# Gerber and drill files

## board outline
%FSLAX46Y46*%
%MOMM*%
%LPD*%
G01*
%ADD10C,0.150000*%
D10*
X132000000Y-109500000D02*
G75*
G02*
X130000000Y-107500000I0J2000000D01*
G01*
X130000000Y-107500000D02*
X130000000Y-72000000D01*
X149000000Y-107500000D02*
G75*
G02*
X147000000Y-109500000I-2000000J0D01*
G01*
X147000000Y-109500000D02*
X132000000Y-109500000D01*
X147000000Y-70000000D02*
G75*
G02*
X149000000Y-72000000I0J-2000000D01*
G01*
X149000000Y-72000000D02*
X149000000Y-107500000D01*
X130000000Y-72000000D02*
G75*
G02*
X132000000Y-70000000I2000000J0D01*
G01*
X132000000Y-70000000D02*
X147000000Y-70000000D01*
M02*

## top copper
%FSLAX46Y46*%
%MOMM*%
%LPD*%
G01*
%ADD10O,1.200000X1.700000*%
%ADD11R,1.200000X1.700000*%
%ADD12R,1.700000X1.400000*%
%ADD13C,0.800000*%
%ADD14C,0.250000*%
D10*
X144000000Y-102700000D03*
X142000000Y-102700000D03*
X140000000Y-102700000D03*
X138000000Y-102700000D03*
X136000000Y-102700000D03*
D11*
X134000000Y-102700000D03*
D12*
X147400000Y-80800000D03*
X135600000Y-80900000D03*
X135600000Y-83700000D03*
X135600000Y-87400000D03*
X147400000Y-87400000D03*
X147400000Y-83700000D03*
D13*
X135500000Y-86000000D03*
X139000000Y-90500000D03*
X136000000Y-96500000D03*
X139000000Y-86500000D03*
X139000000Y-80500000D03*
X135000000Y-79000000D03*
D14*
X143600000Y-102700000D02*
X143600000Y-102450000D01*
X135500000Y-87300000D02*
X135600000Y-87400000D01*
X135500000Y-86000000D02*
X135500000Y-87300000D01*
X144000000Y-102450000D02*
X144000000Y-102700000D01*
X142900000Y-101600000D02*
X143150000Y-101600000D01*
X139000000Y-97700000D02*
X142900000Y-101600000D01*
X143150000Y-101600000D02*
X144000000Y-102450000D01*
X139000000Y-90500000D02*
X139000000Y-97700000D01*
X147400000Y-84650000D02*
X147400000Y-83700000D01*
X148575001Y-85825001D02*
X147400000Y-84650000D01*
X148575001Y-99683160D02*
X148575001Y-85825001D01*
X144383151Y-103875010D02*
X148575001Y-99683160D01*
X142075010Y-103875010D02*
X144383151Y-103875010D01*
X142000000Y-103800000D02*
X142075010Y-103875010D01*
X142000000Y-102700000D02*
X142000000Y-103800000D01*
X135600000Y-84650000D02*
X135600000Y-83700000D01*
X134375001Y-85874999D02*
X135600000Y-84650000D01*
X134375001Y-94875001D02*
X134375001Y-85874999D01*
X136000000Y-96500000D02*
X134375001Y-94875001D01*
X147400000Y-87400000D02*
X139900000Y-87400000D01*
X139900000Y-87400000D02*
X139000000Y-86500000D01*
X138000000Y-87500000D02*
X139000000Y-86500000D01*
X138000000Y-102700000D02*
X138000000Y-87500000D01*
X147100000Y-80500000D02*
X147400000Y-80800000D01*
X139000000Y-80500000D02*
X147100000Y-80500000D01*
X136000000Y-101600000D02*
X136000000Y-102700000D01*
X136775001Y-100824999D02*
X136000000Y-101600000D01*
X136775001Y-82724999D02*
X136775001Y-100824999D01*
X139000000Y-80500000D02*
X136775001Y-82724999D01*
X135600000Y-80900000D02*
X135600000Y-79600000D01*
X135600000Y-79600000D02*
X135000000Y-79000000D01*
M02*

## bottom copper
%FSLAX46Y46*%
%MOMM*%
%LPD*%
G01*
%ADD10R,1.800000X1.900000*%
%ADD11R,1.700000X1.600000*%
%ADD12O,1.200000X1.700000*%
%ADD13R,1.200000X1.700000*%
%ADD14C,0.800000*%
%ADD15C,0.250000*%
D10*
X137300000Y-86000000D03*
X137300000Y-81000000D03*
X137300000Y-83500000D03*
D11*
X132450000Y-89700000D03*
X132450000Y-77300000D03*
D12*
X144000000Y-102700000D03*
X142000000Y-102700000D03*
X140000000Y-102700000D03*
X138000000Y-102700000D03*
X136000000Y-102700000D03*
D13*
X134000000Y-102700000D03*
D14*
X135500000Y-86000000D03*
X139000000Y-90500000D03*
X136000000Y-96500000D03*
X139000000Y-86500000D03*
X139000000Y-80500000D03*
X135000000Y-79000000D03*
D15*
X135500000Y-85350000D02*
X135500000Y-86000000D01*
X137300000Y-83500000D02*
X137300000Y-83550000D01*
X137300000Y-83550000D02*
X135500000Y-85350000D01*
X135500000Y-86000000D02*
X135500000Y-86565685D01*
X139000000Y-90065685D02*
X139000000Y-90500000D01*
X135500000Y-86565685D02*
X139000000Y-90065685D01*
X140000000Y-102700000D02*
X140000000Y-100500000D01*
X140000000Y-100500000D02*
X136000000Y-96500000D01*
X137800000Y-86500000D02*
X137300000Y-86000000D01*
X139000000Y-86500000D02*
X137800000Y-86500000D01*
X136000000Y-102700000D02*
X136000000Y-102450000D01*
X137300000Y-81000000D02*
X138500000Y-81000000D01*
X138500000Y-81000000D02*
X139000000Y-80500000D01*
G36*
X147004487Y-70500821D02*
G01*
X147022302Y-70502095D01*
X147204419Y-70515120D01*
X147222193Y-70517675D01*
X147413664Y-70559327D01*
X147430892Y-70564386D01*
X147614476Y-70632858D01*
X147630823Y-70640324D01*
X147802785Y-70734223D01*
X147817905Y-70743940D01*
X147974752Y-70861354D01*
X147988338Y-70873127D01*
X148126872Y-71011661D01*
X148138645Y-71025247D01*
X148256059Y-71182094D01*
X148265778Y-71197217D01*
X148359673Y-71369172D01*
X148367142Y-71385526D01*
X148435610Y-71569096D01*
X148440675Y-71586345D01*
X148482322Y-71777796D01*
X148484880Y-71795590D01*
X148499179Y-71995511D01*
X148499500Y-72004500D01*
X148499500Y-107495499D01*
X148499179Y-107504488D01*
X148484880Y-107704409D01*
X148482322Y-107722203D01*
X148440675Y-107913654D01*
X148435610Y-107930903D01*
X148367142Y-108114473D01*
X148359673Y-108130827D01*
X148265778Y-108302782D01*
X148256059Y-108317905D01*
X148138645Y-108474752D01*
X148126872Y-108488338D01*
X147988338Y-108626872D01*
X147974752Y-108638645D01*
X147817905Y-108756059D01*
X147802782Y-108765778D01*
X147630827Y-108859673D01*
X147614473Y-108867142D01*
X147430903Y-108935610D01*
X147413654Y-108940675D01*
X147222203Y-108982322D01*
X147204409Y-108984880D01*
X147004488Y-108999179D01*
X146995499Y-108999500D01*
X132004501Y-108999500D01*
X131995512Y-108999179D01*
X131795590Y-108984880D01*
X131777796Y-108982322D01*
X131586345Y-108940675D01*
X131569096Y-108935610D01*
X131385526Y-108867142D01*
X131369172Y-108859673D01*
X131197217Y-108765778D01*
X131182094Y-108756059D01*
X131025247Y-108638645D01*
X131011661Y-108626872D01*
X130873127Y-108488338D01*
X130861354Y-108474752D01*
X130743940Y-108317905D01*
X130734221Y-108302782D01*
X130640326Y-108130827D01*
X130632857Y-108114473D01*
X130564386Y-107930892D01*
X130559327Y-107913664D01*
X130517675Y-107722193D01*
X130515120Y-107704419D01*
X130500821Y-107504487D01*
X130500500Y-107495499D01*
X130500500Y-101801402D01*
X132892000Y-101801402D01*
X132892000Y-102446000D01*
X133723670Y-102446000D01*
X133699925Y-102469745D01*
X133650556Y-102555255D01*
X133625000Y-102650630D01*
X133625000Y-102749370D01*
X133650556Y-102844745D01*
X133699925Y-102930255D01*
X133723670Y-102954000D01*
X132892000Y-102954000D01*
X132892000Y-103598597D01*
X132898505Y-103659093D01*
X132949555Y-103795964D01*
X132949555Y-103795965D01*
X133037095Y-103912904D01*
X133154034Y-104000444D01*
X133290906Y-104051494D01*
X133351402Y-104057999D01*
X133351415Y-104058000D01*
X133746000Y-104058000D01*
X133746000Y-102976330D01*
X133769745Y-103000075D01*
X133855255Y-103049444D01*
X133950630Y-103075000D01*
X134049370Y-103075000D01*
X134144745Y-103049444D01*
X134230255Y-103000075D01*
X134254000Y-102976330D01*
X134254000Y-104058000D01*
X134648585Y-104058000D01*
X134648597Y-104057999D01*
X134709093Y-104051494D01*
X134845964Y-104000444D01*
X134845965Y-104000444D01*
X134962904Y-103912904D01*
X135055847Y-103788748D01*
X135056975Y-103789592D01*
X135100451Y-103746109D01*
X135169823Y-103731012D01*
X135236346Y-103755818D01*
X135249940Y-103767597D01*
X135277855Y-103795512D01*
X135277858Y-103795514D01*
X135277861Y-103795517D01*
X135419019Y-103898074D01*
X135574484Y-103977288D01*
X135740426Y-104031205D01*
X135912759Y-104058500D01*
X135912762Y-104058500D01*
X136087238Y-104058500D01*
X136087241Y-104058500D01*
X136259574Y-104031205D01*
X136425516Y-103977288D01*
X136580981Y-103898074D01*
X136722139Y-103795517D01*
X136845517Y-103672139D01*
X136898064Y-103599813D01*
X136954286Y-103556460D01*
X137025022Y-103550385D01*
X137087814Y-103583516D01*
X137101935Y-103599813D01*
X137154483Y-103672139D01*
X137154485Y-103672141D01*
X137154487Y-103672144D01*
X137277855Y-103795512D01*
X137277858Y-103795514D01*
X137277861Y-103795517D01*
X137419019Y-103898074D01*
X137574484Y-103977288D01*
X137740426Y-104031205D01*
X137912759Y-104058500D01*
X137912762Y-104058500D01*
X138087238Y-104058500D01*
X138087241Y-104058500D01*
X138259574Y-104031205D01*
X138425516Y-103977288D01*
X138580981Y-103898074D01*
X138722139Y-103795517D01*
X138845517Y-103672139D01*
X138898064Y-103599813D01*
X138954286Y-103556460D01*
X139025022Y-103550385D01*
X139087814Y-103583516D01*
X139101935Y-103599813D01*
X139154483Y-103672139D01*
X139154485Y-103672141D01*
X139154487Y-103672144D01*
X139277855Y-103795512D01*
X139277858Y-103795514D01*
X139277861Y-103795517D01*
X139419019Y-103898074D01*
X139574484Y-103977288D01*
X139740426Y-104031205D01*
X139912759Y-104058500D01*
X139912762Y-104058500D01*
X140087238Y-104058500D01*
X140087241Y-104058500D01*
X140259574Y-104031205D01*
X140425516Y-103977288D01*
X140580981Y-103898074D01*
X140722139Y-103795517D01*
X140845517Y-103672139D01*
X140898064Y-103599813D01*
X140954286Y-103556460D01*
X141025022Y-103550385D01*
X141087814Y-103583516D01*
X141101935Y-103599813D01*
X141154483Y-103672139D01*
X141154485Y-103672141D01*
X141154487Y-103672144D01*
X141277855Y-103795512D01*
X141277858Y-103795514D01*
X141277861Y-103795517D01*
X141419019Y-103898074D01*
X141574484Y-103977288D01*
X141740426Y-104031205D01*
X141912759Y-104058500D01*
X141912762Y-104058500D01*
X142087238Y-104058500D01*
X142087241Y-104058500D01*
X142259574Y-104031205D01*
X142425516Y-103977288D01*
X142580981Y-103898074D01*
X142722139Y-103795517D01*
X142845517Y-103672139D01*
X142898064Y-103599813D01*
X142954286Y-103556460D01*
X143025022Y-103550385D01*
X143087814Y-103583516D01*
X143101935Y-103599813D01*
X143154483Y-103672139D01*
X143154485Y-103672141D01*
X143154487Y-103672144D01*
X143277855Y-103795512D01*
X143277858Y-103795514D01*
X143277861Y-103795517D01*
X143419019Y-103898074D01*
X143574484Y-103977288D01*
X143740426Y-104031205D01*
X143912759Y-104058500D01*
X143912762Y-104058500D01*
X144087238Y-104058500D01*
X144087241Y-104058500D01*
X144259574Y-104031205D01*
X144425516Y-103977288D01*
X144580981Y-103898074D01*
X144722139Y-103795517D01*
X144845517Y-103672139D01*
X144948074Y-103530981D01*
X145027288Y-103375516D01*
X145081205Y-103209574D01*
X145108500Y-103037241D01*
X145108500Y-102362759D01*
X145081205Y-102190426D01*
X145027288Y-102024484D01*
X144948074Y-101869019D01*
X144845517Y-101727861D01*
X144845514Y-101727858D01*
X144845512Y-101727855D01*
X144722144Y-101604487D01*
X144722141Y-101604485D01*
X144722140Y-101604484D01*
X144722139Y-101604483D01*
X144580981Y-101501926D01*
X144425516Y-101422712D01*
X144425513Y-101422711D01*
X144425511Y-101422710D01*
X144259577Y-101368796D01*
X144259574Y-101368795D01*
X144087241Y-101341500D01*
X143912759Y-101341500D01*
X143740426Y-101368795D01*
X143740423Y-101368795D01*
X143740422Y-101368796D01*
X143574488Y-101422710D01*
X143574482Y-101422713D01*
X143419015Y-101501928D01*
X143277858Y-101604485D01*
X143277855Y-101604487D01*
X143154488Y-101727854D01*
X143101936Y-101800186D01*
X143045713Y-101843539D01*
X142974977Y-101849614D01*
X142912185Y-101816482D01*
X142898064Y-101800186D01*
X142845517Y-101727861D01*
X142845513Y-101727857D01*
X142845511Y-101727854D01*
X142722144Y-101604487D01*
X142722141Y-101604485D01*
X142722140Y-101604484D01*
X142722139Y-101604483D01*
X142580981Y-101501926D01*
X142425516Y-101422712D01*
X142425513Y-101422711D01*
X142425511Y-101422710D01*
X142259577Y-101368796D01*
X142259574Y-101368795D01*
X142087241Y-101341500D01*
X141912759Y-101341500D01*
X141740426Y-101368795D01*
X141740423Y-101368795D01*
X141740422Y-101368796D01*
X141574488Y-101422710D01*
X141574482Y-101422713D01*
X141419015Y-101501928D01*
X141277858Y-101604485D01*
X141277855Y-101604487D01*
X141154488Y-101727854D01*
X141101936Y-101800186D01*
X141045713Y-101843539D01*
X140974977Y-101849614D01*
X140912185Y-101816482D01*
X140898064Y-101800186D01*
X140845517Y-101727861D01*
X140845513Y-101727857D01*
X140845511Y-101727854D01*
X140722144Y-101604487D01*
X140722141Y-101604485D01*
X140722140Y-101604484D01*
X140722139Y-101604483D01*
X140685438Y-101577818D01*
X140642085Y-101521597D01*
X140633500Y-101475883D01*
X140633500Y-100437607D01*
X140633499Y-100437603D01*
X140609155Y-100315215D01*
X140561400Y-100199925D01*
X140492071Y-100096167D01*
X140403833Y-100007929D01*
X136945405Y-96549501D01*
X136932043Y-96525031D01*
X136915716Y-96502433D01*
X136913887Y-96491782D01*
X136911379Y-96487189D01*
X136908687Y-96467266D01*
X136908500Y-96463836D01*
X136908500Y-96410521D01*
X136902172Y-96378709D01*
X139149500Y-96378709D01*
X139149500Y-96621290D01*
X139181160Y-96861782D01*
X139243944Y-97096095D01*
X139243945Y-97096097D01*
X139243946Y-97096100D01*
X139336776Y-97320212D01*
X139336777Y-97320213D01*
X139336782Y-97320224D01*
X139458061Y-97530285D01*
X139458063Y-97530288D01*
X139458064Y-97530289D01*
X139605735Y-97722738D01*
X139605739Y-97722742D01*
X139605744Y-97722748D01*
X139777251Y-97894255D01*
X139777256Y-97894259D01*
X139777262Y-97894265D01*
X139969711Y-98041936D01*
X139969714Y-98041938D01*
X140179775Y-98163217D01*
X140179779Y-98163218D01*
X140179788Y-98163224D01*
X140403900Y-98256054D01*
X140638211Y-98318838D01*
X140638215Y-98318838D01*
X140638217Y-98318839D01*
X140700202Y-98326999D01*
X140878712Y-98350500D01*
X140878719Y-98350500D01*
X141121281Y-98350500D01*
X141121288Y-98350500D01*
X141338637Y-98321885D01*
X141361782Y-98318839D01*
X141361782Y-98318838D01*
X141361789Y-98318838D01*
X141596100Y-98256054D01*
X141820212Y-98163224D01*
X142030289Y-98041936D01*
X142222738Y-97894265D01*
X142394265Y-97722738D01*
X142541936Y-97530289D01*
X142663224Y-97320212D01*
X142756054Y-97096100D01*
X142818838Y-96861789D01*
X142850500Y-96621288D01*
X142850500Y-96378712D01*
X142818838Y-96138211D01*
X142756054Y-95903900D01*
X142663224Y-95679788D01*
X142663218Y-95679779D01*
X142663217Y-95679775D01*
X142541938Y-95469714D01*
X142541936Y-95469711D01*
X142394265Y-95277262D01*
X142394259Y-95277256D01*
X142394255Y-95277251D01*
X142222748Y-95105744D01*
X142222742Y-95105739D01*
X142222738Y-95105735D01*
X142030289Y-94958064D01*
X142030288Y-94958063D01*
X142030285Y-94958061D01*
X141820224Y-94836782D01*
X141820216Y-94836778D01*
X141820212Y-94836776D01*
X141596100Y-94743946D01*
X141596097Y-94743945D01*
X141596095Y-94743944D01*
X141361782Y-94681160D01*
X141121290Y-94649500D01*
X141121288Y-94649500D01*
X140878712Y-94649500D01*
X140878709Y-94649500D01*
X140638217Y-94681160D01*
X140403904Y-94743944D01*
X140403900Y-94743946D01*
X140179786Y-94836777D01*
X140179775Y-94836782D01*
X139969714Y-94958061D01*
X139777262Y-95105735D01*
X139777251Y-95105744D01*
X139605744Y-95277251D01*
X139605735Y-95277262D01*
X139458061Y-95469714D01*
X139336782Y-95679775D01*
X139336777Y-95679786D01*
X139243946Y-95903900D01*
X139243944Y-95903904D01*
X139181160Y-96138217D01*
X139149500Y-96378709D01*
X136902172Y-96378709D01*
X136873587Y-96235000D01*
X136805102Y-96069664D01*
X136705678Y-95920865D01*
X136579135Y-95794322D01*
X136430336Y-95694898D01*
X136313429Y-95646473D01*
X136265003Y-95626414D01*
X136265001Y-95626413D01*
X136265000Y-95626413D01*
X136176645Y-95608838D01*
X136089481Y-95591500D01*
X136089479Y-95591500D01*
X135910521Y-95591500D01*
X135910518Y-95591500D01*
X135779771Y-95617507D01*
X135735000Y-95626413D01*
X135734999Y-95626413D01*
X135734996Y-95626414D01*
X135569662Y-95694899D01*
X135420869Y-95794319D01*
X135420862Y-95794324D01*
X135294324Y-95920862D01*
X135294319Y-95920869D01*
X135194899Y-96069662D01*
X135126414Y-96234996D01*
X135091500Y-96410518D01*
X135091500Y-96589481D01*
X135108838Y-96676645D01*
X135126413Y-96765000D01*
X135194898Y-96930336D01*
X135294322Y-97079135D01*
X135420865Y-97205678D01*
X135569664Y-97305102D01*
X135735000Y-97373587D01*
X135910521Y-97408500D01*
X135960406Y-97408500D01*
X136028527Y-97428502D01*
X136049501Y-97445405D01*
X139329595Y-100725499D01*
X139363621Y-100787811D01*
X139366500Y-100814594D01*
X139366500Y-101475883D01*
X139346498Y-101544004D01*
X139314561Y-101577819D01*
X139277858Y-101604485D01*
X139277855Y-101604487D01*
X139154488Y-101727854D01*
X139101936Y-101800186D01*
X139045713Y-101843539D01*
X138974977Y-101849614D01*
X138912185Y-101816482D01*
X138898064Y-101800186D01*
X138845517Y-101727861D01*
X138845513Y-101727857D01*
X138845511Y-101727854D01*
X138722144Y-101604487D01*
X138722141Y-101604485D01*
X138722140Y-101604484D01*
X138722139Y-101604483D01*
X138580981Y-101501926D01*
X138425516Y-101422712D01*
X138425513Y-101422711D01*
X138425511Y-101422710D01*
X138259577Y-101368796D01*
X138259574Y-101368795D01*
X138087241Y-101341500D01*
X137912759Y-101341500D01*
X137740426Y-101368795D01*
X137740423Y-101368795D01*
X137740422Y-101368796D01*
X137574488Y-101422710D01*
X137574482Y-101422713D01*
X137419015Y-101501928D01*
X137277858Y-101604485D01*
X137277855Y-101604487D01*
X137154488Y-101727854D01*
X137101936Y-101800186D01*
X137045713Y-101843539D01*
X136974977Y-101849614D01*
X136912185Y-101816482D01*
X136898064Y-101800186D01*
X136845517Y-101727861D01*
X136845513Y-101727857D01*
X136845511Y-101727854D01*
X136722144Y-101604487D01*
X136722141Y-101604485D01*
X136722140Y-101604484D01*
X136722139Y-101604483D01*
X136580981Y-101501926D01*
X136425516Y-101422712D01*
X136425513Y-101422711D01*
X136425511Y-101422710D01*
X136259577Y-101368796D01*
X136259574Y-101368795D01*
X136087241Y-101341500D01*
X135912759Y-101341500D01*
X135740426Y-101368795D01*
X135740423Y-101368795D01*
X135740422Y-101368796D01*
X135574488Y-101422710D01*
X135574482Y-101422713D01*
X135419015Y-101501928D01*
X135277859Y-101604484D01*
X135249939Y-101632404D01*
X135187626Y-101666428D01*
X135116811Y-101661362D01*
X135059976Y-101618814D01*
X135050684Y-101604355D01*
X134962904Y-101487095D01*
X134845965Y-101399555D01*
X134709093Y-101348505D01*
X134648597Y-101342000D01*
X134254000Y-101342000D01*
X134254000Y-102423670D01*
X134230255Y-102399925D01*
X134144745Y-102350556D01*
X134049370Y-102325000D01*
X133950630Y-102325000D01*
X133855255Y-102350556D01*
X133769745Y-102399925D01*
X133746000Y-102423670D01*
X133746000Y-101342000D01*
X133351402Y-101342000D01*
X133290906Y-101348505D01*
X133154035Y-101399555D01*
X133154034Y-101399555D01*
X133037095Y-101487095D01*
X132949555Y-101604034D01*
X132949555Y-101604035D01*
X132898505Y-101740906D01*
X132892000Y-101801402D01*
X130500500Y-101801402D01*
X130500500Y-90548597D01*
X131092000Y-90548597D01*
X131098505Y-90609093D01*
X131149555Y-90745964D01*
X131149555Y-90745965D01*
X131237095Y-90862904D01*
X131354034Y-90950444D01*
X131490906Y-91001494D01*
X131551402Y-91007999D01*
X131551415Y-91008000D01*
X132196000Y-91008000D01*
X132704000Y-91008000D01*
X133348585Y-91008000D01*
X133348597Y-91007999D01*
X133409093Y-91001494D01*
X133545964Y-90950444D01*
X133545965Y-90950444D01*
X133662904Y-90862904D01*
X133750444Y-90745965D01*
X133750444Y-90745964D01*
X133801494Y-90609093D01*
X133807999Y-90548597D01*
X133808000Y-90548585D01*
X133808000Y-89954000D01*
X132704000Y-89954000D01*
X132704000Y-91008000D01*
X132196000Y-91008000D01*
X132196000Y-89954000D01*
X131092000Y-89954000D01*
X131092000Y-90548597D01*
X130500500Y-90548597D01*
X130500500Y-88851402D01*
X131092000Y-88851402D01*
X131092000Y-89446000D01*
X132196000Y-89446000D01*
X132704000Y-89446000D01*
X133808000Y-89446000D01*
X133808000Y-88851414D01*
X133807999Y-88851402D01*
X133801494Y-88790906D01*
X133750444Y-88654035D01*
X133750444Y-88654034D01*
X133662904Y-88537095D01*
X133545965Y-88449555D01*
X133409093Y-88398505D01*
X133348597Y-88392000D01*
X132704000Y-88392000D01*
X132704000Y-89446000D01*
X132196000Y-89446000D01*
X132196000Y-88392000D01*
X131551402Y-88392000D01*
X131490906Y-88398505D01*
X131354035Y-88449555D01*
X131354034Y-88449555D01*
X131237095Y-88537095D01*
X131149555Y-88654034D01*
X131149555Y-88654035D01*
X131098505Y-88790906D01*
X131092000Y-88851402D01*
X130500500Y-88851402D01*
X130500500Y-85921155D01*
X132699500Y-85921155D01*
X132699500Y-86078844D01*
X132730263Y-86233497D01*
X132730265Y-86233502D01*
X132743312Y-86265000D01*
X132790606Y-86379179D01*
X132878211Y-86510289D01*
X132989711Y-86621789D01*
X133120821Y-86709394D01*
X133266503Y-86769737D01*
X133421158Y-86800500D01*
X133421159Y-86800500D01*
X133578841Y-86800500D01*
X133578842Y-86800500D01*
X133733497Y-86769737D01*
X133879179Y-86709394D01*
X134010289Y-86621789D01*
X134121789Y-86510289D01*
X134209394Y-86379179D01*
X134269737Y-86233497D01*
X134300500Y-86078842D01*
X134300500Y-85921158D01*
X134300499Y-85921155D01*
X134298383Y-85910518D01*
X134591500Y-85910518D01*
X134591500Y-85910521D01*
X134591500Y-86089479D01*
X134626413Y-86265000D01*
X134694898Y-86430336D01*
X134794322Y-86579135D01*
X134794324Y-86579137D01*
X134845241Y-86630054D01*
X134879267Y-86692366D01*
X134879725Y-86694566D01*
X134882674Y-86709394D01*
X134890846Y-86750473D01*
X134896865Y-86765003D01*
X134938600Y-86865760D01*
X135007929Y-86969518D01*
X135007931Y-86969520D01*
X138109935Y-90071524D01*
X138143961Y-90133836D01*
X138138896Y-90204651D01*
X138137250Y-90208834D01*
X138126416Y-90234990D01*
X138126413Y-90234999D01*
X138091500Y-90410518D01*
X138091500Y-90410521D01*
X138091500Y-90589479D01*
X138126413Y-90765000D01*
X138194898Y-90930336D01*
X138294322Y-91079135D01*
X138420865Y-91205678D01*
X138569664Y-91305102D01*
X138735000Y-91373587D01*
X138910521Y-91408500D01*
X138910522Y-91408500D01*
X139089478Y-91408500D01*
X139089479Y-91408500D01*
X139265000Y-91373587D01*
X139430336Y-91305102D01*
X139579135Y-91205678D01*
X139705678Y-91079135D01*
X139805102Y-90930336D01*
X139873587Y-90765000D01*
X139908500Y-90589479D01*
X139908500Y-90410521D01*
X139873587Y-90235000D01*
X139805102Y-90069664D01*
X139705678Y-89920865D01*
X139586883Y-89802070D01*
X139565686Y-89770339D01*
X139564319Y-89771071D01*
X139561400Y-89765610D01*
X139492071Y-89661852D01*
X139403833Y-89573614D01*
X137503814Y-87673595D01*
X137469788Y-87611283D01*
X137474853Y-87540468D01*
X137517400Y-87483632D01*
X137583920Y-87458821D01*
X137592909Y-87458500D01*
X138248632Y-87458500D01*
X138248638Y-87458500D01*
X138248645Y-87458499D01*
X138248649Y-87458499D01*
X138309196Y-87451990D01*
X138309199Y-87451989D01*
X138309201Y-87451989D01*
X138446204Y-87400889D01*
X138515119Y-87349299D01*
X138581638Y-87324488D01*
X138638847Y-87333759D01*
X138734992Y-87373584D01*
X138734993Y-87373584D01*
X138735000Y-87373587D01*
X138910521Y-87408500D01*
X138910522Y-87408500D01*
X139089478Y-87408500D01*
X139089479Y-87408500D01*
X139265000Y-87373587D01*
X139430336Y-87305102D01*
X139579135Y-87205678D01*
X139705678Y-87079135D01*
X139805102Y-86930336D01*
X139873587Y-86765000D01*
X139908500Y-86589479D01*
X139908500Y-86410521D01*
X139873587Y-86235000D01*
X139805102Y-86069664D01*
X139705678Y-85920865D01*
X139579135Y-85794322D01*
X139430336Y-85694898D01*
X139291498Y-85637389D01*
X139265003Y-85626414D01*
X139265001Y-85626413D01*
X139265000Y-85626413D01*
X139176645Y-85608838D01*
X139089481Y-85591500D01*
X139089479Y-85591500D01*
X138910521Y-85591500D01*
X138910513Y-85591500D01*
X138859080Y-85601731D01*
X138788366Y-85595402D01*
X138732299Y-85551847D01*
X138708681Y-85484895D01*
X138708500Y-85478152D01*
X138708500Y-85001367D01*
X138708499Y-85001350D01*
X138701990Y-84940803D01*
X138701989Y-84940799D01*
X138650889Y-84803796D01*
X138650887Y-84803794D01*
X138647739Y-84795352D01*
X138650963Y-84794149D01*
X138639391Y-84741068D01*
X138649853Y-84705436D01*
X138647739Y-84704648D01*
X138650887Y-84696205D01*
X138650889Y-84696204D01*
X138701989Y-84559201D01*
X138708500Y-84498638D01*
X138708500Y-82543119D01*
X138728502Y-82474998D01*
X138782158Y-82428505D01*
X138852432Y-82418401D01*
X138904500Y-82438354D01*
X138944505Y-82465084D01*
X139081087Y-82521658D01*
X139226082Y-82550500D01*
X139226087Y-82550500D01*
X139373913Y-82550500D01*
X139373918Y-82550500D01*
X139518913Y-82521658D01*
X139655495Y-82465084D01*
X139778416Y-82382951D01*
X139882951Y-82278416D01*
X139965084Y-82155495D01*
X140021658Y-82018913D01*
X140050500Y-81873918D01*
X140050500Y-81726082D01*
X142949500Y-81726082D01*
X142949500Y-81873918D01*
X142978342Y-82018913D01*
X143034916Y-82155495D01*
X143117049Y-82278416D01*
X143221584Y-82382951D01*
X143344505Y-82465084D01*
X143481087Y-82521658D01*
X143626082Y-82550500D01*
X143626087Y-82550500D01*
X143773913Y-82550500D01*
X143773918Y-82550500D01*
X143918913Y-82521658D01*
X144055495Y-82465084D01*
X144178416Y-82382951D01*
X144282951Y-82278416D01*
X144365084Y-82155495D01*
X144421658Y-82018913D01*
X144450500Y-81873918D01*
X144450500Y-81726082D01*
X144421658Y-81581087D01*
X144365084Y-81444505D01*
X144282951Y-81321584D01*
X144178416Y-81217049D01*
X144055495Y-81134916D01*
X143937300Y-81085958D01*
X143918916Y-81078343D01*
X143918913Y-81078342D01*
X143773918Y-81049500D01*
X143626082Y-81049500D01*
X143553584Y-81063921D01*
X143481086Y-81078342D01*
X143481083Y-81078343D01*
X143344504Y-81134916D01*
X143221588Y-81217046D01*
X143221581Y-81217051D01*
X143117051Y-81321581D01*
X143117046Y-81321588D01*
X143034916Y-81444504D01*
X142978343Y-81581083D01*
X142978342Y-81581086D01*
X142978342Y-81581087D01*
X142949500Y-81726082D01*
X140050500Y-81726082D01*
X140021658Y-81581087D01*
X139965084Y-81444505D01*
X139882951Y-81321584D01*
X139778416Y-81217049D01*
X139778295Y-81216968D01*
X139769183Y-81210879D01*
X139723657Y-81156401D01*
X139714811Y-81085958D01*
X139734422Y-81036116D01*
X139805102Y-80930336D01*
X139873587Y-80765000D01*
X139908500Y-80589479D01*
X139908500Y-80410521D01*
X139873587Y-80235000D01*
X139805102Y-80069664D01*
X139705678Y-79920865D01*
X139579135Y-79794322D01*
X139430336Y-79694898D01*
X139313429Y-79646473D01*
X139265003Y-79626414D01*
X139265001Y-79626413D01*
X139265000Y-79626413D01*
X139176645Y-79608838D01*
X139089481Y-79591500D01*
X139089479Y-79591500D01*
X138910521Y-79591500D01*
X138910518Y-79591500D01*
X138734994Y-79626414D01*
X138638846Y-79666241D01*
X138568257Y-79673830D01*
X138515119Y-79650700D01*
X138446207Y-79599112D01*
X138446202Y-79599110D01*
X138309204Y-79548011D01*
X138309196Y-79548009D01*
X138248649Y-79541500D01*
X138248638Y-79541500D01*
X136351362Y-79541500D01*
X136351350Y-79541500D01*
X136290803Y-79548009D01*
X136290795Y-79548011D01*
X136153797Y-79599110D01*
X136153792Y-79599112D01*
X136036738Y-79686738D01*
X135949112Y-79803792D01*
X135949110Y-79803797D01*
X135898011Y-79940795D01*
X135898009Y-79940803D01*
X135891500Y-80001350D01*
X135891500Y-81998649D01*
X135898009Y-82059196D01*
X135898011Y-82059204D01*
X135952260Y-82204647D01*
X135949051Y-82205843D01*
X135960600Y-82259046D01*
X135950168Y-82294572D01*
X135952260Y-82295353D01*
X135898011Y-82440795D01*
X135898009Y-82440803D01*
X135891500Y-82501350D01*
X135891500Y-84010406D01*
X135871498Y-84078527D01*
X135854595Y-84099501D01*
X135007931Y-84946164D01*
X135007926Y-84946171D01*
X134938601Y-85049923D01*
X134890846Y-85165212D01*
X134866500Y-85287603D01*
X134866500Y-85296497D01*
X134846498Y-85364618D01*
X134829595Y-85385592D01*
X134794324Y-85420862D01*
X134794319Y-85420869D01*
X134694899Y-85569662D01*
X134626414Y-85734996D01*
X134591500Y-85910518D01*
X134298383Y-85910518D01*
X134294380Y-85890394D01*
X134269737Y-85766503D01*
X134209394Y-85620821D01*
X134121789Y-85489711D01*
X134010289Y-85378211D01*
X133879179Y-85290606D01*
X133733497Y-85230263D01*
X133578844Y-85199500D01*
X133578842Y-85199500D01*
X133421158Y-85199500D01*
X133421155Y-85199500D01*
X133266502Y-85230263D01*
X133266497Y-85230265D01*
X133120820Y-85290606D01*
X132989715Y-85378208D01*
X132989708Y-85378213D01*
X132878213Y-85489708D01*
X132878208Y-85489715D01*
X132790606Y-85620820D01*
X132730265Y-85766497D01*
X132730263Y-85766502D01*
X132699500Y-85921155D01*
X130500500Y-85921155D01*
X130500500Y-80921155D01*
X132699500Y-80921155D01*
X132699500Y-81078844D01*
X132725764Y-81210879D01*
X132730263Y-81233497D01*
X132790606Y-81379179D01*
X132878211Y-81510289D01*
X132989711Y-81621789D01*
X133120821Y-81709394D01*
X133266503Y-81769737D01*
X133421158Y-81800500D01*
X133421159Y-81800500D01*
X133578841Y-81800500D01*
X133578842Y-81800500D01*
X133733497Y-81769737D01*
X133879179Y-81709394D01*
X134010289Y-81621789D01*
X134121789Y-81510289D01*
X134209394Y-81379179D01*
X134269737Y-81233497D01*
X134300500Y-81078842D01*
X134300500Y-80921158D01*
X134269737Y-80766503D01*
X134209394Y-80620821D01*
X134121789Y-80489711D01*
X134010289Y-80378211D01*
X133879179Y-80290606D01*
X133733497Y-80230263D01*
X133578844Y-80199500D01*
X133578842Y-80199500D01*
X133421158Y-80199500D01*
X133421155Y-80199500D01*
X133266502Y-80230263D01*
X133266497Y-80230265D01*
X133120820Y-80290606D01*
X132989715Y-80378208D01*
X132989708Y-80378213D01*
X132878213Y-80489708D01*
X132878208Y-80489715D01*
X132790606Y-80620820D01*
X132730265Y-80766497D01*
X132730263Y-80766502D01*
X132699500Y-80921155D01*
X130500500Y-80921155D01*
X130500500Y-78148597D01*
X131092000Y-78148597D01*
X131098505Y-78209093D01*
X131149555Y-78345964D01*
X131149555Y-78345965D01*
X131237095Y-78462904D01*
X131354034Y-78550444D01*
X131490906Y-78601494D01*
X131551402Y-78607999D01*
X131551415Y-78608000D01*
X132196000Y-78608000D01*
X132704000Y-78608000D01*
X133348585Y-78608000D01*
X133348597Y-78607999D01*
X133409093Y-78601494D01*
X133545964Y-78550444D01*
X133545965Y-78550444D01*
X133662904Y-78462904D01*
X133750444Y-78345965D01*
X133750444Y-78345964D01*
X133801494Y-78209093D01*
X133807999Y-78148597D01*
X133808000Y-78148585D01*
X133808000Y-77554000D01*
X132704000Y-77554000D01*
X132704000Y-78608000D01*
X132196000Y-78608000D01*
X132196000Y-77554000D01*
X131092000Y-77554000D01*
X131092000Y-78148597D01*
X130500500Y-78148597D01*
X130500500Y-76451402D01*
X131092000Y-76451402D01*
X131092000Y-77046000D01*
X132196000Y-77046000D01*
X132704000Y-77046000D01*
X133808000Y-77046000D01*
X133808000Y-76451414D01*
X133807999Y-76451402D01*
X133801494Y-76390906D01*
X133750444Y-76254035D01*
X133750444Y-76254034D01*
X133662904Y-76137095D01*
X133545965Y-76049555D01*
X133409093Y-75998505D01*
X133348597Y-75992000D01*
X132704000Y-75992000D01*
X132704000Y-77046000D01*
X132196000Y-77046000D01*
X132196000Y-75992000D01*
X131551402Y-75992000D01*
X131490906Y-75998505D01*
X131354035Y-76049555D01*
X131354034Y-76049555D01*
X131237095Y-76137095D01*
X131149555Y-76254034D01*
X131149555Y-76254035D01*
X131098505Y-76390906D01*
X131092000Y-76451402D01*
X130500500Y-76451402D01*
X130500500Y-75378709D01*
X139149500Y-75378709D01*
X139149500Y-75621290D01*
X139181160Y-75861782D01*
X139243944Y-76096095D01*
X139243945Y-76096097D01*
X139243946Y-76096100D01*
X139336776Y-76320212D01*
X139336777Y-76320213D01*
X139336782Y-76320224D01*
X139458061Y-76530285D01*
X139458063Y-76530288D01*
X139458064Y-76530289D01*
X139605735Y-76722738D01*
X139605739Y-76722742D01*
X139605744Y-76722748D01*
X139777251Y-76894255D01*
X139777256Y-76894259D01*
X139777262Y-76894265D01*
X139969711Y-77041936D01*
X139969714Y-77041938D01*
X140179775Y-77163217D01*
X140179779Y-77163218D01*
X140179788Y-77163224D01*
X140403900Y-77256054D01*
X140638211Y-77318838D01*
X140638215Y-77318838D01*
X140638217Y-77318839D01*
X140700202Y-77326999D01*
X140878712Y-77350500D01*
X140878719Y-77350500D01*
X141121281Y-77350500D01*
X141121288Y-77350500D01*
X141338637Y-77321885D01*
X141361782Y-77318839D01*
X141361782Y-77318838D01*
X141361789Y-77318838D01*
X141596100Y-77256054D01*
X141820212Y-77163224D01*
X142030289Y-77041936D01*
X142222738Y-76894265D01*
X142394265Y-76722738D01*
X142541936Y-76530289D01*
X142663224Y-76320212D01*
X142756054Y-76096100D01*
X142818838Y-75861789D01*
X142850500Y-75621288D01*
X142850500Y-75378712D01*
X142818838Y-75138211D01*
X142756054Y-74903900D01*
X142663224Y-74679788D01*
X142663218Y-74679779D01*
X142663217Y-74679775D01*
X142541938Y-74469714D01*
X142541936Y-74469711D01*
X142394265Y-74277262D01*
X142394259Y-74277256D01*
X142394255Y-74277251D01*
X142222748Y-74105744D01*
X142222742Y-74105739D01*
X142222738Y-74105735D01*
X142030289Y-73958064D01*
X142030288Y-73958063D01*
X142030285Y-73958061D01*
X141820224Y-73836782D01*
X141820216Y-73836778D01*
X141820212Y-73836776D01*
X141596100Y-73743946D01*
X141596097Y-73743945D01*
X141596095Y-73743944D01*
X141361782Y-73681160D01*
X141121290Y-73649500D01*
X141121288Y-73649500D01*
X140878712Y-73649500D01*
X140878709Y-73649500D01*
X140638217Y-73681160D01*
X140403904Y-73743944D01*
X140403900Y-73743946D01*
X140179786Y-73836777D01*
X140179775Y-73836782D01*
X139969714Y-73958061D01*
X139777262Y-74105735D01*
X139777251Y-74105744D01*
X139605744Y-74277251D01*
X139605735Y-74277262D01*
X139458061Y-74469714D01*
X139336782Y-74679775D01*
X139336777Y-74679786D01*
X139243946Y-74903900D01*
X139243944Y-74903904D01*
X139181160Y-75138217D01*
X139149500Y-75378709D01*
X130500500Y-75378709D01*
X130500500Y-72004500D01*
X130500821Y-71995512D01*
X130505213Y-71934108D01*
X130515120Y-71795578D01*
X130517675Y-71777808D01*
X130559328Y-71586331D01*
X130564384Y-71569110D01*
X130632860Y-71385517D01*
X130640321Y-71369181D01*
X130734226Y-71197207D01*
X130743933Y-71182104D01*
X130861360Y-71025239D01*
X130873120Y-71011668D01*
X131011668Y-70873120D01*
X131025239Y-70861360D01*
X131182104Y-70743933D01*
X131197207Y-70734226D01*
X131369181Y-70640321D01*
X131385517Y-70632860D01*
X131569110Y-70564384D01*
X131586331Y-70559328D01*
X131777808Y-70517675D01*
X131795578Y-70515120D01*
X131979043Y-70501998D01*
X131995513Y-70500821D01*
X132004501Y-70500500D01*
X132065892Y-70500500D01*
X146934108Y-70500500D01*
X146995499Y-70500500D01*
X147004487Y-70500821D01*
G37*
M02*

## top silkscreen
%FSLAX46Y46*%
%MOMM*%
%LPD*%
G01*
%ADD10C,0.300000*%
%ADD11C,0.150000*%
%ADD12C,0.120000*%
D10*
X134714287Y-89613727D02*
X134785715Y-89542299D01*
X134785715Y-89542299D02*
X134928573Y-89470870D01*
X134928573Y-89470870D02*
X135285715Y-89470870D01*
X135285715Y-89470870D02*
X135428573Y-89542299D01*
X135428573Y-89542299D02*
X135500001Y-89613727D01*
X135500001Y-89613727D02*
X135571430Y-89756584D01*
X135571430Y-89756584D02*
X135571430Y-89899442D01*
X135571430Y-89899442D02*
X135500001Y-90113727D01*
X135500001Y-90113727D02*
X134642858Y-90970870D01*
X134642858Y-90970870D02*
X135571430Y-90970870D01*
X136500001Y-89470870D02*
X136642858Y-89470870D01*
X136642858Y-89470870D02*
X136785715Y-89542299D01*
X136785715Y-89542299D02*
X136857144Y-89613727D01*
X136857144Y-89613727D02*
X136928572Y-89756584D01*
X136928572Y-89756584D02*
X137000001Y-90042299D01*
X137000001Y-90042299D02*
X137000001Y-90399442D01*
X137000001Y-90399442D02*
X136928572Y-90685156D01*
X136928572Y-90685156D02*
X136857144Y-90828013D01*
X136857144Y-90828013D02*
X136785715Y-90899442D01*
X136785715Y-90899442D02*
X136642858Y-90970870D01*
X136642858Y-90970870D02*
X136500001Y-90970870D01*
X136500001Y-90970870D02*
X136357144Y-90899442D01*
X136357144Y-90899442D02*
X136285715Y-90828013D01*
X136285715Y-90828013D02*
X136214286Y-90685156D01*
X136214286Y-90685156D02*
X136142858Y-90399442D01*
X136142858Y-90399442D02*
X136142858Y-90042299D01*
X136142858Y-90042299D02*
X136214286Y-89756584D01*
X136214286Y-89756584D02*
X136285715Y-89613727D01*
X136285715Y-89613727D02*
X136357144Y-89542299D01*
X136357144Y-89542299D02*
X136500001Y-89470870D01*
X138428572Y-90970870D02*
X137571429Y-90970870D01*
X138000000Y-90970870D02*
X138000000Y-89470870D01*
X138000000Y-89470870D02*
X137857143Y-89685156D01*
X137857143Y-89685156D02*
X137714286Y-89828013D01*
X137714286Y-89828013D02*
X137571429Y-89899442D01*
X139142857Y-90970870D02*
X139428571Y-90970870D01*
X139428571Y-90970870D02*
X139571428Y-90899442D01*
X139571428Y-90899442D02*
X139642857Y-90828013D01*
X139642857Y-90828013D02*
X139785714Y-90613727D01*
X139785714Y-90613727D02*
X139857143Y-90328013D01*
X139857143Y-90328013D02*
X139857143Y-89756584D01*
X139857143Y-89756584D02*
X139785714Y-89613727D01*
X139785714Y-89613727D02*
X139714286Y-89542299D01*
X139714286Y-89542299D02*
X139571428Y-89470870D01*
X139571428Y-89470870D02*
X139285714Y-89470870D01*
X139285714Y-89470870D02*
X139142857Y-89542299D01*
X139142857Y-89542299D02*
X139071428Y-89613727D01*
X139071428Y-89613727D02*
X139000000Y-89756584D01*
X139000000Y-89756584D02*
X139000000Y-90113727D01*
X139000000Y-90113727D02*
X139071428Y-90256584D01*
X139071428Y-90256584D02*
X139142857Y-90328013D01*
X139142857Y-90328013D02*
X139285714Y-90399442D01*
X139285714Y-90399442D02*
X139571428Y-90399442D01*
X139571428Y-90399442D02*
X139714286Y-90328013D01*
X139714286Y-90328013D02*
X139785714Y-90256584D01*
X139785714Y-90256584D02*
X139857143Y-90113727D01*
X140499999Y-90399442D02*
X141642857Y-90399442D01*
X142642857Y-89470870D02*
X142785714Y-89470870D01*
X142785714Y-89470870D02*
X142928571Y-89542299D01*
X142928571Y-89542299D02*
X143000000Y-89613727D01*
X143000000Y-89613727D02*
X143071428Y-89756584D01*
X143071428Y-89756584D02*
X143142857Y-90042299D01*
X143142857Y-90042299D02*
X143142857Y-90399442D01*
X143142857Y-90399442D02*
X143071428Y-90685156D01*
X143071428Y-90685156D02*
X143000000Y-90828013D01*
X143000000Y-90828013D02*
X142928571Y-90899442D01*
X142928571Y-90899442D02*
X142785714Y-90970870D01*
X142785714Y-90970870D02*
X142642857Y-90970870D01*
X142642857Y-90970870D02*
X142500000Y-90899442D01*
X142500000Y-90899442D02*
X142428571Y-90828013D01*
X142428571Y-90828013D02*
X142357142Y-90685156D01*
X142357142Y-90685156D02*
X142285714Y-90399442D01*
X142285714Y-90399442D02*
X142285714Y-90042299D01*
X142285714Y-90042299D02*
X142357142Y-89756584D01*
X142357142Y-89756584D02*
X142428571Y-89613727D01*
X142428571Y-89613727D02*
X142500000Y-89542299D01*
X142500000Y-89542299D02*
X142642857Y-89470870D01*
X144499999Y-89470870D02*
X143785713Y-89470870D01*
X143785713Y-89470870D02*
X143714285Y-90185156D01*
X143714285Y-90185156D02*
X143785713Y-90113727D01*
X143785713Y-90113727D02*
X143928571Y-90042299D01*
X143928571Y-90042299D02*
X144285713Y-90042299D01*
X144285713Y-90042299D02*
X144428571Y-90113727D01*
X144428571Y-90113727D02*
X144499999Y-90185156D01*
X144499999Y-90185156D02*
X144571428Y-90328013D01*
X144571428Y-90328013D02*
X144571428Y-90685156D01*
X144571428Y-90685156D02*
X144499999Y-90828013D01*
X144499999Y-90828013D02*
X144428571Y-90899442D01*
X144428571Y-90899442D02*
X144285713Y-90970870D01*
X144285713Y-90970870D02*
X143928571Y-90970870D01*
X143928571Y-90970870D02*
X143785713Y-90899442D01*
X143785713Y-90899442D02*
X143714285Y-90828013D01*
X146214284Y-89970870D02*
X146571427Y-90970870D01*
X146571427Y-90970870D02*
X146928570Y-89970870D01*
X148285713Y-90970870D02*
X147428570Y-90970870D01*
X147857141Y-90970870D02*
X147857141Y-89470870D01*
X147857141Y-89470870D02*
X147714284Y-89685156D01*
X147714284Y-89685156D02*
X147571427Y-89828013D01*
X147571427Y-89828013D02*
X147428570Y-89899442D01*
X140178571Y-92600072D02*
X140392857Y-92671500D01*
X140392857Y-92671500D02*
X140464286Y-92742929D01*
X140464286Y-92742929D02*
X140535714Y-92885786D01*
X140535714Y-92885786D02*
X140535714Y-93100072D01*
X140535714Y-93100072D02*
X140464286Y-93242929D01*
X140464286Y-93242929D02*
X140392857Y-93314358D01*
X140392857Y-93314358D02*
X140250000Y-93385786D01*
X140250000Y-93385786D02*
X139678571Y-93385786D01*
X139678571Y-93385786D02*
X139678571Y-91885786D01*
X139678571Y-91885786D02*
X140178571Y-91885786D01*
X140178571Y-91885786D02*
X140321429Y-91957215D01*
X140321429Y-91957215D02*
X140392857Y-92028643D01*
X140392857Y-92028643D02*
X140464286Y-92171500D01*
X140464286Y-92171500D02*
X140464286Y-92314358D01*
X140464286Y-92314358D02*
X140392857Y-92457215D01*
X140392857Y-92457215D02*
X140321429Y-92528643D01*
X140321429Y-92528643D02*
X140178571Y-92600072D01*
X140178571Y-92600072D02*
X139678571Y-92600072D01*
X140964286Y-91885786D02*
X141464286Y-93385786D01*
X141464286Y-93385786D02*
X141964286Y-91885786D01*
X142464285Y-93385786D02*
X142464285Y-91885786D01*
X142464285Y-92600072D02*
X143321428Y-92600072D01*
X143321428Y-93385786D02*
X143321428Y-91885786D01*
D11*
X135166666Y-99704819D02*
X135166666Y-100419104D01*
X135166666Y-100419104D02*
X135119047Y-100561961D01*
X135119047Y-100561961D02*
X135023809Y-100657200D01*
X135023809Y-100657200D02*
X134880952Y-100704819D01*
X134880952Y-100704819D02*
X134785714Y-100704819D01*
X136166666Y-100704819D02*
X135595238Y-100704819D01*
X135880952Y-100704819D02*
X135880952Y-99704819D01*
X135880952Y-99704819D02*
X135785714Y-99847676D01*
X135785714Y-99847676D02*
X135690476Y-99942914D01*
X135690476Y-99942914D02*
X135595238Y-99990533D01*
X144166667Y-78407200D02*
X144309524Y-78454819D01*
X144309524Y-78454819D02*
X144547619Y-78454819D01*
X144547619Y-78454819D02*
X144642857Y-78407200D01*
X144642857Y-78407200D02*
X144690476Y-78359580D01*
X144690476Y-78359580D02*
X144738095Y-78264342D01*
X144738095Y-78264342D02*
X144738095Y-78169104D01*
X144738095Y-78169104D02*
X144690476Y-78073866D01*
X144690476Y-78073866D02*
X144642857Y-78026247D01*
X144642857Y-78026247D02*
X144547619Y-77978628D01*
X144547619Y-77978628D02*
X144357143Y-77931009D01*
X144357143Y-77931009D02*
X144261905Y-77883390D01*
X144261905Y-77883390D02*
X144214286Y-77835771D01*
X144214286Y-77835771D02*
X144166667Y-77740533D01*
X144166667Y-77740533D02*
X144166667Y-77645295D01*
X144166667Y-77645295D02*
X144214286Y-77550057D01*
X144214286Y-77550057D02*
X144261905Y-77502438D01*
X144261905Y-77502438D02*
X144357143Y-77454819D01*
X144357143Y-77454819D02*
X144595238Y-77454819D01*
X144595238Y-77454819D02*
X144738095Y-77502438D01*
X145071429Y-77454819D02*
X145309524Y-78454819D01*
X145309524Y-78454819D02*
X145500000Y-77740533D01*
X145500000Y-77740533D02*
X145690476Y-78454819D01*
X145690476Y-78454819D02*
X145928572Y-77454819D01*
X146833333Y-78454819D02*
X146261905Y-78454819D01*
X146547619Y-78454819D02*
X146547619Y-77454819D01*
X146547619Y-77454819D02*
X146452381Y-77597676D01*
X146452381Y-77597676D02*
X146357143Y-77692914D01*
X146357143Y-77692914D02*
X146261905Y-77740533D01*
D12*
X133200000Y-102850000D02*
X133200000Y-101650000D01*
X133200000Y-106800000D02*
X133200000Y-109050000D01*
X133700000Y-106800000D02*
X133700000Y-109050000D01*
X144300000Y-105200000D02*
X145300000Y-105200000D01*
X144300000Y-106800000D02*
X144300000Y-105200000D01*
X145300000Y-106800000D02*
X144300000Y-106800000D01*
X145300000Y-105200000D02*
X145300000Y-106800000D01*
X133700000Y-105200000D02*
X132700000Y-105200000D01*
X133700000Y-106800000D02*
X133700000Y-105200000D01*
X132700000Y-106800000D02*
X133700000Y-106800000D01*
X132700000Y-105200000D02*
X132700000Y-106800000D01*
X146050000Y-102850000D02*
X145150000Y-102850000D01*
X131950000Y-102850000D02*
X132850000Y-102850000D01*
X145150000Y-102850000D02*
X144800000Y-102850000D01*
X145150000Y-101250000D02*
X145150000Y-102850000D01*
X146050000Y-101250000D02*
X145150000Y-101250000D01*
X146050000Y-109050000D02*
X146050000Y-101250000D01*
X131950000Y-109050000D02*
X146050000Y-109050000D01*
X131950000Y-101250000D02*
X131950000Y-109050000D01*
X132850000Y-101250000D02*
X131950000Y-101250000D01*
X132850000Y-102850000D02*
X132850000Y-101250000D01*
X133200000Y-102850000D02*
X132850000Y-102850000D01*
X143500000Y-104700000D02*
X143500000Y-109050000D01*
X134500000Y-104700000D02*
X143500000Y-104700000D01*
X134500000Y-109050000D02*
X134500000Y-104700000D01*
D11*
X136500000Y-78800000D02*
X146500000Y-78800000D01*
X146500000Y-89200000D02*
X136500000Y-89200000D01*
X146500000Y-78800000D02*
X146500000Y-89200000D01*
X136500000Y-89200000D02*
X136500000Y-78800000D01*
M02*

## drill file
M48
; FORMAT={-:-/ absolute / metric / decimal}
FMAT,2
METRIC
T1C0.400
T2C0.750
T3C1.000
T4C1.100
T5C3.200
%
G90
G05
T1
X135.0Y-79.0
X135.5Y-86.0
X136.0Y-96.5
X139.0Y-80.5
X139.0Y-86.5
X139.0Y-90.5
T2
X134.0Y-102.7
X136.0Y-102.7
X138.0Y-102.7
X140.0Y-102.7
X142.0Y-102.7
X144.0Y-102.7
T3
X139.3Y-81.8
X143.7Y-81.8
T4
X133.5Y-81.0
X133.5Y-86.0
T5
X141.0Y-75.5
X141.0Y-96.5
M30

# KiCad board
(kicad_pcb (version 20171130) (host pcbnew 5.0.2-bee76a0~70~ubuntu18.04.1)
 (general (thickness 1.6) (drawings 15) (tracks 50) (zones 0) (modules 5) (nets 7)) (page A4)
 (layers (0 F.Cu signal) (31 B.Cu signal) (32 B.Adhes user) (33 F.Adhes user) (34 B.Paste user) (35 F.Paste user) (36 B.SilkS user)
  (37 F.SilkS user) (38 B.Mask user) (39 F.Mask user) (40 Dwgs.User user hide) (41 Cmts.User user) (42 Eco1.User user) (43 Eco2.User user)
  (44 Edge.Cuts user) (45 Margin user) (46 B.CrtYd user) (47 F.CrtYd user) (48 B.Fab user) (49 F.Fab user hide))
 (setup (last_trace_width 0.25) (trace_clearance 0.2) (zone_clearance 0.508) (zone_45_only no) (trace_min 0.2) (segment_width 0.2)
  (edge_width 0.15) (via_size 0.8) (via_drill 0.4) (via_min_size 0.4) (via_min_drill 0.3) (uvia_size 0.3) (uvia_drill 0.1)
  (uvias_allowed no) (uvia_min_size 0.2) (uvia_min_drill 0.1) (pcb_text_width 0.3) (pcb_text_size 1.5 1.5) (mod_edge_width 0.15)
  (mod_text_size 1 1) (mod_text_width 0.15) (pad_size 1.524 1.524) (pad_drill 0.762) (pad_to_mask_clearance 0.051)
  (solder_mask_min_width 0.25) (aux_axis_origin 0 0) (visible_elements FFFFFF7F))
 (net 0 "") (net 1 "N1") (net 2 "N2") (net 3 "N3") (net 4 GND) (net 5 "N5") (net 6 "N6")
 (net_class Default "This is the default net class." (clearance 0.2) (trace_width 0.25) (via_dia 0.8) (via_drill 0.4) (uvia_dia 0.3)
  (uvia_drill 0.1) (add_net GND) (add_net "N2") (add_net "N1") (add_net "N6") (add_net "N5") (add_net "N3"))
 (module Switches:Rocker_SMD (layer B.Cu) (at 133.5 83.5 270)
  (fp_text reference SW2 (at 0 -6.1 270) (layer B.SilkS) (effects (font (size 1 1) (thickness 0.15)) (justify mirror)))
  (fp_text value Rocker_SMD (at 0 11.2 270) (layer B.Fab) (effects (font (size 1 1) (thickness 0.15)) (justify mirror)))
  (pad 5 smd rect (at 2.5 -3.8 270) (size 1.9 1.8) (layers B.Cu B.Paste B.Mask) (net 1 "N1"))
  (pad 3 smd rect (at -2.5 -3.8 270) (size 1.9 1.8) (layers B.Cu B.Paste B.Mask) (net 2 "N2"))
  (pad 4 smd rect (at 0 -3.8 270) (size 1.9 1.8) (layers B.Cu B.Paste B.Mask) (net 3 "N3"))
  (pad 2 smd rect (at 6.2 1.05 270) (size 1.6 1.7) (layers B.Cu B.Paste B.Mask) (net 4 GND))
  (pad 2 smd rect (at -6.2 1.05 270) (size 1.6 1.7) (layers B.Cu B.Paste B.Mask) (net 4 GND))
  (pad "" np_thru_hole circle (at 2.5 0 270) (size 1.1 1.1) (drill 1.1) (layers *.Cu *.Mask))
  (pad "" np_thru_hole circle (at -2.5 0 270) (size 1.1 1.1) (drill 1.1) (layers *.Cu *.Mask)))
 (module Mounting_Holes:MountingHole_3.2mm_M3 (layer F.Cu) (at 141 96.5)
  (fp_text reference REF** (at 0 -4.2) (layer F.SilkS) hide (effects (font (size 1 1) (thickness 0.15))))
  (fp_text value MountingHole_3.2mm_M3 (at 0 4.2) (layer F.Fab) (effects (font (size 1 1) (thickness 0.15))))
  (pad 1 np_thru_hole circle (at 0 0) (size 3.2 3.2) (drill 3.2) (layers *.Cu *.Mask)))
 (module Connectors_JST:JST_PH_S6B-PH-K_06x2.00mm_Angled (layer F.Cu) (at 134 102.7)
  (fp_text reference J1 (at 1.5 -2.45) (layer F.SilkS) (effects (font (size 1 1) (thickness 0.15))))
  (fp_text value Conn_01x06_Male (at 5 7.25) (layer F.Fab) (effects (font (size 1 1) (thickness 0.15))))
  (fp_line (start -0.8 0.15) (end -0.8 -1.05) (layer F.SilkS) (width 0.12))
  (fp_line (start -0.8 4.1) (end -0.8 6.35) (layer F.SilkS) (width 0.12))
  (fp_line (start -0.3 4.1) (end -0.3 6.35) (layer F.SilkS) (width 0.12))
  (fp_line (start 10.3 2.5) (end 11.3 2.5) (layer F.SilkS) (width 0.12))
  (fp_line (start 10.3 4.1) (end 10.3 2.5) (layer F.SilkS) (width 0.12))
  (fp_line (start 11.3 4.1) (end 10.3 4.1) (layer F.SilkS) (width 0.12))
  (fp_line (start 11.3 2.5) (end 11.3 4.1) (layer F.SilkS) (width 0.12))
  (fp_line (start -0.3 2.5) (end -1.3 2.5) (layer F.SilkS) (width 0.12))
  (fp_line (start -0.3 4.1) (end -0.3 2.5) (layer F.SilkS) (width 0.12))
  (fp_line (start -1.3 4.1) (end -0.3 4.1) (layer F.SilkS) (width 0.12))
  (fp_line (start -1.3 2.5) (end -1.3 4.1) (layer F.SilkS) (width 0.12))
  (fp_line (start 12.05 0.15) (end 11.15 0.15) (layer F.SilkS) (width 0.12))
  (fp_line (start -2.05 0.15) (end -1.15 0.15) (layer F.SilkS) (width 0.12))
  (fp_line (start 11.15 0.15) (end 10.8 0.15) (layer F.SilkS) (width 0.12))
  (fp_line (start 11.15 -1.45) (end 11.15 0.15) (layer F.SilkS) (width 0.12))
  (fp_line (start 12.05 -1.45) (end 11.15 -1.45) (layer F.SilkS) (width 0.12))
  (fp_line (start 12.05 6.35) (end 12.05 -1.45) (layer F.SilkS) (width 0.12))
  (fp_line (start -2.05 6.35) (end 12.05 6.35) (layer F.SilkS) (width 0.12))
  (fp_line (start -2.05 -1.45) (end -2.05 6.35) (layer F.SilkS) (width 0.12))
  (fp_line (start -1.15 -1.45) (end -2.05 -1.45) (layer F.SilkS) (width 0.12))
  (fp_line (start -1.15 0.15) (end -1.15 -1.45) (layer F.SilkS) (width 0.12))
  (fp_line (start -0.8 0.15) (end -1.15 0.15) (layer F.SilkS) (width 0.12))
  (fp_line (start 9.5 2) (end 9.5 6.35) (layer F.SilkS) (width 0.12))
  (fp_line (start 0.5 2) (end 9.5 2) (layer F.SilkS) (width 0.12))
  (fp_line (start 0.5 6.35) (end 0.5 2) (layer F.SilkS) (width 0.12))
  (pad 6 thru_hole oval (at 10 0) (size 1.2 1.7) (drill 0.75) (layers *.Cu *.Mask) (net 3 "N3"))
  (pad 5 thru_hole oval (at 8 0) (size 1.2 1.7) (drill 0.75) (layers *.Cu *.Mask) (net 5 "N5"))
  (pad 4 thru_hole oval (at 6 0) (size 1.2 1.7) (drill 0.75) (layers *.Cu *.Mask) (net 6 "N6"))
  (pad 3 thru_hole oval (at 4 0) (size 1.2 1.7) (drill 0.75) (layers *.Cu *.Mask) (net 1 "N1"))
  (pad 2 thru_hole oval (at 2 0) (size 1.2 1.7) (drill 0.75) (layers *.Cu *.Mask) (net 2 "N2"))
  (pad 1 thru_hole rect (at 0 0) (size 1.2 1.7) (drill 0.75) (layers *.Cu *.Mask) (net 4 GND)))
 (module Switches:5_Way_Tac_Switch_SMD (layer F.Cu) (at 141.5 84)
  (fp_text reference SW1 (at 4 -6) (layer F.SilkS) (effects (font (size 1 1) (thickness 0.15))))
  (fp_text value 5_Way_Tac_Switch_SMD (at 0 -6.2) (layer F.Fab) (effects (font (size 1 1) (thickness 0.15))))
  (fp_line (start -5 -5.2) (end 5 -5.2) (layer F.SilkS) (width 0.15))
  (fp_line (start 5 5.2) (end -5 5.2) (layer F.SilkS) (width 0.15))
  (fp_line (start 5 -5.2) (end 5 5.2) (layer F.SilkS) (width 0.15))
  (fp_line (start -5 5.2) (end -5 -5.2) (layer F.SilkS) (width 0.15))
  (pad 4 smd rect (at 5.9 -3.2) (size 1.7 1.4) (layers F.Cu F.Paste F.Mask) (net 2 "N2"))
  (pad 1 smd rect (at -5.9 -3.1) (size 1.7 1.4) (layers F.Cu F.Paste F.Mask) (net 4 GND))
  (pad 2 smd rect (at -5.9 -0.3) (size 1.7 1.4) (layers F.Cu F.Paste F.Mask) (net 6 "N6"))
  (pad 3 smd rect (at -5.9 3.4) (size 1.7 1.4) (layers F.Cu F.Paste F.Mask) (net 3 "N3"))
  (pad 6 smd rect (at 5.9 3.4) (size 1.7 1.4) (layers F.Cu F.Paste F.Mask) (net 1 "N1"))
  (pad 5 smd rect (at 5.9 -0.3) (size 1.7 1.4) (layers F.Cu F.Paste F.Mask) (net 5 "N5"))
  (pad "" np_thru_hole circle (at -2.2 -2.2) (size 1 1) (drill 1) (layers *.Cu *.Mask))
  (pad "" np_thru_hole circle (at 2.2 -2.2) (size 1 1) (drill 1) (layers *.Cu *.Mask)))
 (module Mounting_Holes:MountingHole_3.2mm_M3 (layer F.Cu) (at 141 75.5)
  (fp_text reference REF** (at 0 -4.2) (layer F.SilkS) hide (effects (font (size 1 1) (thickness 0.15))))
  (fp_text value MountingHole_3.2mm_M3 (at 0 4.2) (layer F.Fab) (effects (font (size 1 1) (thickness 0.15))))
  (pad 1 np_thru_hole circle (at 0 0) (size 3.2 3.2) (drill 3.2) (layers *.Cu *.Mask)))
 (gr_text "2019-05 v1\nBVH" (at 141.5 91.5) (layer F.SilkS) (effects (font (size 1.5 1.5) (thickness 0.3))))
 (gr_arc (start 132 107.5) (end 130 107.5) (angle -90) (layer Edge.Cuts) (width 0.15))
 (gr_line (start 130 107.5) (end 130 72) (layer Edge.Cuts) (width 0.15))
 (gr_arc (start 147 107.5) (end 147 109.5) (angle -90) (layer Edge.Cuts) (width 0.15))
 (gr_line (start 147 109.5) (end 132 109.5) (layer Edge.Cuts) (width 0.15))
 (gr_arc (start 147 72) (end 149 72) (angle -90) (layer Edge.Cuts) (width 0.15))
 (gr_line (start 149 72) (end 149 107.5) (layer Edge.Cuts) (width 0.15))
 (gr_arc (start 132 72) (end 132 70) (angle -90) (layer Edge.Cuts) (width 0.15))
 (gr_line (start 132 70) (end 147 70) (layer Edge.Cuts) (width 0.15))
 (segment (start 143.6 102.7) (end 143.6 102.45) (width 0.25) (layer F.Cu) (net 3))
 (segment (start 135.5 85.35) (end 135.5 86) (width 0.25) (layer B.Cu) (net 3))
 (via (at 135.5 86) (size 0.8) (drill 0.4) (layers F.Cu B.Cu) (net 3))
 (segment (start 137.3 83.5) (end 137.3 83.55) (width 0.25) (layer B.Cu) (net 3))
 (segment (start 137.3 83.55) (end 135.5 85.35) (width 0.25) (layer B.Cu) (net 3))
 (segment (start 135.5 87.3) (end 135.6 87.4) (width 0.25) (layer F.Cu) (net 3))
 (segment (start 135.5 86) (end 135.5 87.3) (width 0.25) (layer F.Cu) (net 3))
 (via (at 139 90.5) (size 0.8) (drill 0.4) (layers F.Cu B.Cu) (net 3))
 (segment (start 135.5 86) (end 135.5 86.565685) (width 0.25) (layer B.Cu) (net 3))
 (segment (start 139 90.065685) (end 139 90.5) (width 0.25) (layer B.Cu) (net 3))
 (segment (start 135.5 86.565685) (end 139 90.065685) (width 0.25) (layer B.Cu) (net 3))
 (segment (start 144 102.45) (end 144 102.7) (width 0.25) (layer F.Cu) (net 3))
 (segment (start 142.9 101.6) (end 143.15 101.6) (width 0.25) (layer F.Cu) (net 3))
 (segment (start 139 97.7) (end 142.9 101.6) (width 0.25) (layer F.Cu) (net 3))
 (segment (start 143.15 101.6) (end 144 102.45) (width 0.25) (layer F.Cu) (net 3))
 (segment (start 139 90.5) (end 139 97.7) (width 0.25) (layer F.Cu) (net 3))
 (segment (start 147.4 84.65) (end 147.4 83.7) (width 0.25) (layer F.Cu) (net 5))
 (segment (start 148.575001 85.825001) (end 147.4 84.65) (width 0.25) (layer F.Cu) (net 5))
 (segment (start 148.575001 99.68316) (end 148.575001 85.825001) (width 0.25) (layer F.Cu) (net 5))
 (segment (start 144.383151 103.87501) (end 148.575001 99.68316) (width 0.25) (layer F.Cu) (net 5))
 (segment (start 142.07501 103.87501) (end 144.383151 103.87501) (width 0.25) (layer F.Cu) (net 5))
 (segment (start 142 103.8) (end 142.07501 103.87501) (width 0.25) (layer F.Cu) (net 5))
 (segment (start 142 102.7) (end 142 103.8) (width 0.25) (layer F.Cu) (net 5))
 (via (at 136 96.5) (size 0.8) (drill 0.4) (layers F.Cu B.Cu) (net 6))
 (segment (start 140 102.7) (end 140 100.5) (width 0.25) (layer B.Cu) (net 6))
 (segment (start 140 100.5) (end 136 96.5) (width 0.25) (layer B.Cu) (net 6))
 (segment (start 135.6 84.65) (end 135.6 83.7) (width 0.25) (layer F.Cu) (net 6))
 (segment (start 134.375001 85.874999) (end 135.6 84.65) (width 0.25) (layer F.Cu) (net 6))
 (segment (start 134.375001 94.875001) (end 134.375001 85.874999) (width 0.25) (layer F.Cu) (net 6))
 (segment (start 136 96.5) (end 134.375001 94.875001) (width 0.25) (layer F.Cu) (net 6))
 (via (at 139 86.5) (size 0.8) (drill 0.4) (layers F.Cu B.Cu) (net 1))
 (segment (start 147.4 87.4) (end 139.9 87.4) (width 0.25) (layer F.Cu) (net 1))
 (segment (start 139.9 87.4) (end 139 86.5) (width 0.25) (layer F.Cu) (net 1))
 (segment (start 137.8 86.5) (end 137.3 86) (width 0.25) (layer B.Cu) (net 1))
 (segment (start 139 86.5) (end 137.8 86.5) (width 0.25) (layer B.Cu) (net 1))
 (segment (start 138 87.5) (end 139 86.5) (width 0.25) (layer F.Cu) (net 1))
 (segment (start 138 102.7) (end 138 87.5) (width 0.25) (layer F.Cu) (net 1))
 (segment (start 136 102.7) (end 136 102.45) (width 0.25) (layer B.Cu) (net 2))
 (via (at 139 80.5) (size 0.8) (drill 0.4) (layers F.Cu B.Cu) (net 2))
 (segment (start 137.3 81) (end 138.5 81) (width 0.25) (layer B.Cu) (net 2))
 (segment (start 138.5 81) (end 139 80.5) (width 0.25) (layer B.Cu) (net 2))
 (segment (start 147.1 80.5) (end 147.4 80.8) (width 0.25) (layer F.Cu) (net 2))
 (segment (start 139 80.5) (end 147.1 80.5) (width 0.25) (layer F.Cu) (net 2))
 (segment (start 136 101.6) (end 136 102.7) (width 0.25) (layer F.Cu) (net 2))
 (segment (start 136.775001 100.824999) (end 136 101.6) (width 0.25) (layer F.Cu) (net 2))
 (segment (start 136.775001 82.724999) (end 136.775001 100.824999) (width 0.25) (layer F.Cu) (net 2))
 (segment (start 139 80.5) (end 136.775001 82.724999) (width 0.25) (layer F.Cu) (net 2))
 (via (at 135 79) (size 0.8) (drill 0.4) (layers F.Cu B.Cu) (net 4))
 (segment (start 135.6 80.9) (end 135.6 79.6) (width 0.25) (layer F.Cu) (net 4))
 (segment (start 135.6 79.6) (end 135 79) (width 0.25) (layer F.Cu) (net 4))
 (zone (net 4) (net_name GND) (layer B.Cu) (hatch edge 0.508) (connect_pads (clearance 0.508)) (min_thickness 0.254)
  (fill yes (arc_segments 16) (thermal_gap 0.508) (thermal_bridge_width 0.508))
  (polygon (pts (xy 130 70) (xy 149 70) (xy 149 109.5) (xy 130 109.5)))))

